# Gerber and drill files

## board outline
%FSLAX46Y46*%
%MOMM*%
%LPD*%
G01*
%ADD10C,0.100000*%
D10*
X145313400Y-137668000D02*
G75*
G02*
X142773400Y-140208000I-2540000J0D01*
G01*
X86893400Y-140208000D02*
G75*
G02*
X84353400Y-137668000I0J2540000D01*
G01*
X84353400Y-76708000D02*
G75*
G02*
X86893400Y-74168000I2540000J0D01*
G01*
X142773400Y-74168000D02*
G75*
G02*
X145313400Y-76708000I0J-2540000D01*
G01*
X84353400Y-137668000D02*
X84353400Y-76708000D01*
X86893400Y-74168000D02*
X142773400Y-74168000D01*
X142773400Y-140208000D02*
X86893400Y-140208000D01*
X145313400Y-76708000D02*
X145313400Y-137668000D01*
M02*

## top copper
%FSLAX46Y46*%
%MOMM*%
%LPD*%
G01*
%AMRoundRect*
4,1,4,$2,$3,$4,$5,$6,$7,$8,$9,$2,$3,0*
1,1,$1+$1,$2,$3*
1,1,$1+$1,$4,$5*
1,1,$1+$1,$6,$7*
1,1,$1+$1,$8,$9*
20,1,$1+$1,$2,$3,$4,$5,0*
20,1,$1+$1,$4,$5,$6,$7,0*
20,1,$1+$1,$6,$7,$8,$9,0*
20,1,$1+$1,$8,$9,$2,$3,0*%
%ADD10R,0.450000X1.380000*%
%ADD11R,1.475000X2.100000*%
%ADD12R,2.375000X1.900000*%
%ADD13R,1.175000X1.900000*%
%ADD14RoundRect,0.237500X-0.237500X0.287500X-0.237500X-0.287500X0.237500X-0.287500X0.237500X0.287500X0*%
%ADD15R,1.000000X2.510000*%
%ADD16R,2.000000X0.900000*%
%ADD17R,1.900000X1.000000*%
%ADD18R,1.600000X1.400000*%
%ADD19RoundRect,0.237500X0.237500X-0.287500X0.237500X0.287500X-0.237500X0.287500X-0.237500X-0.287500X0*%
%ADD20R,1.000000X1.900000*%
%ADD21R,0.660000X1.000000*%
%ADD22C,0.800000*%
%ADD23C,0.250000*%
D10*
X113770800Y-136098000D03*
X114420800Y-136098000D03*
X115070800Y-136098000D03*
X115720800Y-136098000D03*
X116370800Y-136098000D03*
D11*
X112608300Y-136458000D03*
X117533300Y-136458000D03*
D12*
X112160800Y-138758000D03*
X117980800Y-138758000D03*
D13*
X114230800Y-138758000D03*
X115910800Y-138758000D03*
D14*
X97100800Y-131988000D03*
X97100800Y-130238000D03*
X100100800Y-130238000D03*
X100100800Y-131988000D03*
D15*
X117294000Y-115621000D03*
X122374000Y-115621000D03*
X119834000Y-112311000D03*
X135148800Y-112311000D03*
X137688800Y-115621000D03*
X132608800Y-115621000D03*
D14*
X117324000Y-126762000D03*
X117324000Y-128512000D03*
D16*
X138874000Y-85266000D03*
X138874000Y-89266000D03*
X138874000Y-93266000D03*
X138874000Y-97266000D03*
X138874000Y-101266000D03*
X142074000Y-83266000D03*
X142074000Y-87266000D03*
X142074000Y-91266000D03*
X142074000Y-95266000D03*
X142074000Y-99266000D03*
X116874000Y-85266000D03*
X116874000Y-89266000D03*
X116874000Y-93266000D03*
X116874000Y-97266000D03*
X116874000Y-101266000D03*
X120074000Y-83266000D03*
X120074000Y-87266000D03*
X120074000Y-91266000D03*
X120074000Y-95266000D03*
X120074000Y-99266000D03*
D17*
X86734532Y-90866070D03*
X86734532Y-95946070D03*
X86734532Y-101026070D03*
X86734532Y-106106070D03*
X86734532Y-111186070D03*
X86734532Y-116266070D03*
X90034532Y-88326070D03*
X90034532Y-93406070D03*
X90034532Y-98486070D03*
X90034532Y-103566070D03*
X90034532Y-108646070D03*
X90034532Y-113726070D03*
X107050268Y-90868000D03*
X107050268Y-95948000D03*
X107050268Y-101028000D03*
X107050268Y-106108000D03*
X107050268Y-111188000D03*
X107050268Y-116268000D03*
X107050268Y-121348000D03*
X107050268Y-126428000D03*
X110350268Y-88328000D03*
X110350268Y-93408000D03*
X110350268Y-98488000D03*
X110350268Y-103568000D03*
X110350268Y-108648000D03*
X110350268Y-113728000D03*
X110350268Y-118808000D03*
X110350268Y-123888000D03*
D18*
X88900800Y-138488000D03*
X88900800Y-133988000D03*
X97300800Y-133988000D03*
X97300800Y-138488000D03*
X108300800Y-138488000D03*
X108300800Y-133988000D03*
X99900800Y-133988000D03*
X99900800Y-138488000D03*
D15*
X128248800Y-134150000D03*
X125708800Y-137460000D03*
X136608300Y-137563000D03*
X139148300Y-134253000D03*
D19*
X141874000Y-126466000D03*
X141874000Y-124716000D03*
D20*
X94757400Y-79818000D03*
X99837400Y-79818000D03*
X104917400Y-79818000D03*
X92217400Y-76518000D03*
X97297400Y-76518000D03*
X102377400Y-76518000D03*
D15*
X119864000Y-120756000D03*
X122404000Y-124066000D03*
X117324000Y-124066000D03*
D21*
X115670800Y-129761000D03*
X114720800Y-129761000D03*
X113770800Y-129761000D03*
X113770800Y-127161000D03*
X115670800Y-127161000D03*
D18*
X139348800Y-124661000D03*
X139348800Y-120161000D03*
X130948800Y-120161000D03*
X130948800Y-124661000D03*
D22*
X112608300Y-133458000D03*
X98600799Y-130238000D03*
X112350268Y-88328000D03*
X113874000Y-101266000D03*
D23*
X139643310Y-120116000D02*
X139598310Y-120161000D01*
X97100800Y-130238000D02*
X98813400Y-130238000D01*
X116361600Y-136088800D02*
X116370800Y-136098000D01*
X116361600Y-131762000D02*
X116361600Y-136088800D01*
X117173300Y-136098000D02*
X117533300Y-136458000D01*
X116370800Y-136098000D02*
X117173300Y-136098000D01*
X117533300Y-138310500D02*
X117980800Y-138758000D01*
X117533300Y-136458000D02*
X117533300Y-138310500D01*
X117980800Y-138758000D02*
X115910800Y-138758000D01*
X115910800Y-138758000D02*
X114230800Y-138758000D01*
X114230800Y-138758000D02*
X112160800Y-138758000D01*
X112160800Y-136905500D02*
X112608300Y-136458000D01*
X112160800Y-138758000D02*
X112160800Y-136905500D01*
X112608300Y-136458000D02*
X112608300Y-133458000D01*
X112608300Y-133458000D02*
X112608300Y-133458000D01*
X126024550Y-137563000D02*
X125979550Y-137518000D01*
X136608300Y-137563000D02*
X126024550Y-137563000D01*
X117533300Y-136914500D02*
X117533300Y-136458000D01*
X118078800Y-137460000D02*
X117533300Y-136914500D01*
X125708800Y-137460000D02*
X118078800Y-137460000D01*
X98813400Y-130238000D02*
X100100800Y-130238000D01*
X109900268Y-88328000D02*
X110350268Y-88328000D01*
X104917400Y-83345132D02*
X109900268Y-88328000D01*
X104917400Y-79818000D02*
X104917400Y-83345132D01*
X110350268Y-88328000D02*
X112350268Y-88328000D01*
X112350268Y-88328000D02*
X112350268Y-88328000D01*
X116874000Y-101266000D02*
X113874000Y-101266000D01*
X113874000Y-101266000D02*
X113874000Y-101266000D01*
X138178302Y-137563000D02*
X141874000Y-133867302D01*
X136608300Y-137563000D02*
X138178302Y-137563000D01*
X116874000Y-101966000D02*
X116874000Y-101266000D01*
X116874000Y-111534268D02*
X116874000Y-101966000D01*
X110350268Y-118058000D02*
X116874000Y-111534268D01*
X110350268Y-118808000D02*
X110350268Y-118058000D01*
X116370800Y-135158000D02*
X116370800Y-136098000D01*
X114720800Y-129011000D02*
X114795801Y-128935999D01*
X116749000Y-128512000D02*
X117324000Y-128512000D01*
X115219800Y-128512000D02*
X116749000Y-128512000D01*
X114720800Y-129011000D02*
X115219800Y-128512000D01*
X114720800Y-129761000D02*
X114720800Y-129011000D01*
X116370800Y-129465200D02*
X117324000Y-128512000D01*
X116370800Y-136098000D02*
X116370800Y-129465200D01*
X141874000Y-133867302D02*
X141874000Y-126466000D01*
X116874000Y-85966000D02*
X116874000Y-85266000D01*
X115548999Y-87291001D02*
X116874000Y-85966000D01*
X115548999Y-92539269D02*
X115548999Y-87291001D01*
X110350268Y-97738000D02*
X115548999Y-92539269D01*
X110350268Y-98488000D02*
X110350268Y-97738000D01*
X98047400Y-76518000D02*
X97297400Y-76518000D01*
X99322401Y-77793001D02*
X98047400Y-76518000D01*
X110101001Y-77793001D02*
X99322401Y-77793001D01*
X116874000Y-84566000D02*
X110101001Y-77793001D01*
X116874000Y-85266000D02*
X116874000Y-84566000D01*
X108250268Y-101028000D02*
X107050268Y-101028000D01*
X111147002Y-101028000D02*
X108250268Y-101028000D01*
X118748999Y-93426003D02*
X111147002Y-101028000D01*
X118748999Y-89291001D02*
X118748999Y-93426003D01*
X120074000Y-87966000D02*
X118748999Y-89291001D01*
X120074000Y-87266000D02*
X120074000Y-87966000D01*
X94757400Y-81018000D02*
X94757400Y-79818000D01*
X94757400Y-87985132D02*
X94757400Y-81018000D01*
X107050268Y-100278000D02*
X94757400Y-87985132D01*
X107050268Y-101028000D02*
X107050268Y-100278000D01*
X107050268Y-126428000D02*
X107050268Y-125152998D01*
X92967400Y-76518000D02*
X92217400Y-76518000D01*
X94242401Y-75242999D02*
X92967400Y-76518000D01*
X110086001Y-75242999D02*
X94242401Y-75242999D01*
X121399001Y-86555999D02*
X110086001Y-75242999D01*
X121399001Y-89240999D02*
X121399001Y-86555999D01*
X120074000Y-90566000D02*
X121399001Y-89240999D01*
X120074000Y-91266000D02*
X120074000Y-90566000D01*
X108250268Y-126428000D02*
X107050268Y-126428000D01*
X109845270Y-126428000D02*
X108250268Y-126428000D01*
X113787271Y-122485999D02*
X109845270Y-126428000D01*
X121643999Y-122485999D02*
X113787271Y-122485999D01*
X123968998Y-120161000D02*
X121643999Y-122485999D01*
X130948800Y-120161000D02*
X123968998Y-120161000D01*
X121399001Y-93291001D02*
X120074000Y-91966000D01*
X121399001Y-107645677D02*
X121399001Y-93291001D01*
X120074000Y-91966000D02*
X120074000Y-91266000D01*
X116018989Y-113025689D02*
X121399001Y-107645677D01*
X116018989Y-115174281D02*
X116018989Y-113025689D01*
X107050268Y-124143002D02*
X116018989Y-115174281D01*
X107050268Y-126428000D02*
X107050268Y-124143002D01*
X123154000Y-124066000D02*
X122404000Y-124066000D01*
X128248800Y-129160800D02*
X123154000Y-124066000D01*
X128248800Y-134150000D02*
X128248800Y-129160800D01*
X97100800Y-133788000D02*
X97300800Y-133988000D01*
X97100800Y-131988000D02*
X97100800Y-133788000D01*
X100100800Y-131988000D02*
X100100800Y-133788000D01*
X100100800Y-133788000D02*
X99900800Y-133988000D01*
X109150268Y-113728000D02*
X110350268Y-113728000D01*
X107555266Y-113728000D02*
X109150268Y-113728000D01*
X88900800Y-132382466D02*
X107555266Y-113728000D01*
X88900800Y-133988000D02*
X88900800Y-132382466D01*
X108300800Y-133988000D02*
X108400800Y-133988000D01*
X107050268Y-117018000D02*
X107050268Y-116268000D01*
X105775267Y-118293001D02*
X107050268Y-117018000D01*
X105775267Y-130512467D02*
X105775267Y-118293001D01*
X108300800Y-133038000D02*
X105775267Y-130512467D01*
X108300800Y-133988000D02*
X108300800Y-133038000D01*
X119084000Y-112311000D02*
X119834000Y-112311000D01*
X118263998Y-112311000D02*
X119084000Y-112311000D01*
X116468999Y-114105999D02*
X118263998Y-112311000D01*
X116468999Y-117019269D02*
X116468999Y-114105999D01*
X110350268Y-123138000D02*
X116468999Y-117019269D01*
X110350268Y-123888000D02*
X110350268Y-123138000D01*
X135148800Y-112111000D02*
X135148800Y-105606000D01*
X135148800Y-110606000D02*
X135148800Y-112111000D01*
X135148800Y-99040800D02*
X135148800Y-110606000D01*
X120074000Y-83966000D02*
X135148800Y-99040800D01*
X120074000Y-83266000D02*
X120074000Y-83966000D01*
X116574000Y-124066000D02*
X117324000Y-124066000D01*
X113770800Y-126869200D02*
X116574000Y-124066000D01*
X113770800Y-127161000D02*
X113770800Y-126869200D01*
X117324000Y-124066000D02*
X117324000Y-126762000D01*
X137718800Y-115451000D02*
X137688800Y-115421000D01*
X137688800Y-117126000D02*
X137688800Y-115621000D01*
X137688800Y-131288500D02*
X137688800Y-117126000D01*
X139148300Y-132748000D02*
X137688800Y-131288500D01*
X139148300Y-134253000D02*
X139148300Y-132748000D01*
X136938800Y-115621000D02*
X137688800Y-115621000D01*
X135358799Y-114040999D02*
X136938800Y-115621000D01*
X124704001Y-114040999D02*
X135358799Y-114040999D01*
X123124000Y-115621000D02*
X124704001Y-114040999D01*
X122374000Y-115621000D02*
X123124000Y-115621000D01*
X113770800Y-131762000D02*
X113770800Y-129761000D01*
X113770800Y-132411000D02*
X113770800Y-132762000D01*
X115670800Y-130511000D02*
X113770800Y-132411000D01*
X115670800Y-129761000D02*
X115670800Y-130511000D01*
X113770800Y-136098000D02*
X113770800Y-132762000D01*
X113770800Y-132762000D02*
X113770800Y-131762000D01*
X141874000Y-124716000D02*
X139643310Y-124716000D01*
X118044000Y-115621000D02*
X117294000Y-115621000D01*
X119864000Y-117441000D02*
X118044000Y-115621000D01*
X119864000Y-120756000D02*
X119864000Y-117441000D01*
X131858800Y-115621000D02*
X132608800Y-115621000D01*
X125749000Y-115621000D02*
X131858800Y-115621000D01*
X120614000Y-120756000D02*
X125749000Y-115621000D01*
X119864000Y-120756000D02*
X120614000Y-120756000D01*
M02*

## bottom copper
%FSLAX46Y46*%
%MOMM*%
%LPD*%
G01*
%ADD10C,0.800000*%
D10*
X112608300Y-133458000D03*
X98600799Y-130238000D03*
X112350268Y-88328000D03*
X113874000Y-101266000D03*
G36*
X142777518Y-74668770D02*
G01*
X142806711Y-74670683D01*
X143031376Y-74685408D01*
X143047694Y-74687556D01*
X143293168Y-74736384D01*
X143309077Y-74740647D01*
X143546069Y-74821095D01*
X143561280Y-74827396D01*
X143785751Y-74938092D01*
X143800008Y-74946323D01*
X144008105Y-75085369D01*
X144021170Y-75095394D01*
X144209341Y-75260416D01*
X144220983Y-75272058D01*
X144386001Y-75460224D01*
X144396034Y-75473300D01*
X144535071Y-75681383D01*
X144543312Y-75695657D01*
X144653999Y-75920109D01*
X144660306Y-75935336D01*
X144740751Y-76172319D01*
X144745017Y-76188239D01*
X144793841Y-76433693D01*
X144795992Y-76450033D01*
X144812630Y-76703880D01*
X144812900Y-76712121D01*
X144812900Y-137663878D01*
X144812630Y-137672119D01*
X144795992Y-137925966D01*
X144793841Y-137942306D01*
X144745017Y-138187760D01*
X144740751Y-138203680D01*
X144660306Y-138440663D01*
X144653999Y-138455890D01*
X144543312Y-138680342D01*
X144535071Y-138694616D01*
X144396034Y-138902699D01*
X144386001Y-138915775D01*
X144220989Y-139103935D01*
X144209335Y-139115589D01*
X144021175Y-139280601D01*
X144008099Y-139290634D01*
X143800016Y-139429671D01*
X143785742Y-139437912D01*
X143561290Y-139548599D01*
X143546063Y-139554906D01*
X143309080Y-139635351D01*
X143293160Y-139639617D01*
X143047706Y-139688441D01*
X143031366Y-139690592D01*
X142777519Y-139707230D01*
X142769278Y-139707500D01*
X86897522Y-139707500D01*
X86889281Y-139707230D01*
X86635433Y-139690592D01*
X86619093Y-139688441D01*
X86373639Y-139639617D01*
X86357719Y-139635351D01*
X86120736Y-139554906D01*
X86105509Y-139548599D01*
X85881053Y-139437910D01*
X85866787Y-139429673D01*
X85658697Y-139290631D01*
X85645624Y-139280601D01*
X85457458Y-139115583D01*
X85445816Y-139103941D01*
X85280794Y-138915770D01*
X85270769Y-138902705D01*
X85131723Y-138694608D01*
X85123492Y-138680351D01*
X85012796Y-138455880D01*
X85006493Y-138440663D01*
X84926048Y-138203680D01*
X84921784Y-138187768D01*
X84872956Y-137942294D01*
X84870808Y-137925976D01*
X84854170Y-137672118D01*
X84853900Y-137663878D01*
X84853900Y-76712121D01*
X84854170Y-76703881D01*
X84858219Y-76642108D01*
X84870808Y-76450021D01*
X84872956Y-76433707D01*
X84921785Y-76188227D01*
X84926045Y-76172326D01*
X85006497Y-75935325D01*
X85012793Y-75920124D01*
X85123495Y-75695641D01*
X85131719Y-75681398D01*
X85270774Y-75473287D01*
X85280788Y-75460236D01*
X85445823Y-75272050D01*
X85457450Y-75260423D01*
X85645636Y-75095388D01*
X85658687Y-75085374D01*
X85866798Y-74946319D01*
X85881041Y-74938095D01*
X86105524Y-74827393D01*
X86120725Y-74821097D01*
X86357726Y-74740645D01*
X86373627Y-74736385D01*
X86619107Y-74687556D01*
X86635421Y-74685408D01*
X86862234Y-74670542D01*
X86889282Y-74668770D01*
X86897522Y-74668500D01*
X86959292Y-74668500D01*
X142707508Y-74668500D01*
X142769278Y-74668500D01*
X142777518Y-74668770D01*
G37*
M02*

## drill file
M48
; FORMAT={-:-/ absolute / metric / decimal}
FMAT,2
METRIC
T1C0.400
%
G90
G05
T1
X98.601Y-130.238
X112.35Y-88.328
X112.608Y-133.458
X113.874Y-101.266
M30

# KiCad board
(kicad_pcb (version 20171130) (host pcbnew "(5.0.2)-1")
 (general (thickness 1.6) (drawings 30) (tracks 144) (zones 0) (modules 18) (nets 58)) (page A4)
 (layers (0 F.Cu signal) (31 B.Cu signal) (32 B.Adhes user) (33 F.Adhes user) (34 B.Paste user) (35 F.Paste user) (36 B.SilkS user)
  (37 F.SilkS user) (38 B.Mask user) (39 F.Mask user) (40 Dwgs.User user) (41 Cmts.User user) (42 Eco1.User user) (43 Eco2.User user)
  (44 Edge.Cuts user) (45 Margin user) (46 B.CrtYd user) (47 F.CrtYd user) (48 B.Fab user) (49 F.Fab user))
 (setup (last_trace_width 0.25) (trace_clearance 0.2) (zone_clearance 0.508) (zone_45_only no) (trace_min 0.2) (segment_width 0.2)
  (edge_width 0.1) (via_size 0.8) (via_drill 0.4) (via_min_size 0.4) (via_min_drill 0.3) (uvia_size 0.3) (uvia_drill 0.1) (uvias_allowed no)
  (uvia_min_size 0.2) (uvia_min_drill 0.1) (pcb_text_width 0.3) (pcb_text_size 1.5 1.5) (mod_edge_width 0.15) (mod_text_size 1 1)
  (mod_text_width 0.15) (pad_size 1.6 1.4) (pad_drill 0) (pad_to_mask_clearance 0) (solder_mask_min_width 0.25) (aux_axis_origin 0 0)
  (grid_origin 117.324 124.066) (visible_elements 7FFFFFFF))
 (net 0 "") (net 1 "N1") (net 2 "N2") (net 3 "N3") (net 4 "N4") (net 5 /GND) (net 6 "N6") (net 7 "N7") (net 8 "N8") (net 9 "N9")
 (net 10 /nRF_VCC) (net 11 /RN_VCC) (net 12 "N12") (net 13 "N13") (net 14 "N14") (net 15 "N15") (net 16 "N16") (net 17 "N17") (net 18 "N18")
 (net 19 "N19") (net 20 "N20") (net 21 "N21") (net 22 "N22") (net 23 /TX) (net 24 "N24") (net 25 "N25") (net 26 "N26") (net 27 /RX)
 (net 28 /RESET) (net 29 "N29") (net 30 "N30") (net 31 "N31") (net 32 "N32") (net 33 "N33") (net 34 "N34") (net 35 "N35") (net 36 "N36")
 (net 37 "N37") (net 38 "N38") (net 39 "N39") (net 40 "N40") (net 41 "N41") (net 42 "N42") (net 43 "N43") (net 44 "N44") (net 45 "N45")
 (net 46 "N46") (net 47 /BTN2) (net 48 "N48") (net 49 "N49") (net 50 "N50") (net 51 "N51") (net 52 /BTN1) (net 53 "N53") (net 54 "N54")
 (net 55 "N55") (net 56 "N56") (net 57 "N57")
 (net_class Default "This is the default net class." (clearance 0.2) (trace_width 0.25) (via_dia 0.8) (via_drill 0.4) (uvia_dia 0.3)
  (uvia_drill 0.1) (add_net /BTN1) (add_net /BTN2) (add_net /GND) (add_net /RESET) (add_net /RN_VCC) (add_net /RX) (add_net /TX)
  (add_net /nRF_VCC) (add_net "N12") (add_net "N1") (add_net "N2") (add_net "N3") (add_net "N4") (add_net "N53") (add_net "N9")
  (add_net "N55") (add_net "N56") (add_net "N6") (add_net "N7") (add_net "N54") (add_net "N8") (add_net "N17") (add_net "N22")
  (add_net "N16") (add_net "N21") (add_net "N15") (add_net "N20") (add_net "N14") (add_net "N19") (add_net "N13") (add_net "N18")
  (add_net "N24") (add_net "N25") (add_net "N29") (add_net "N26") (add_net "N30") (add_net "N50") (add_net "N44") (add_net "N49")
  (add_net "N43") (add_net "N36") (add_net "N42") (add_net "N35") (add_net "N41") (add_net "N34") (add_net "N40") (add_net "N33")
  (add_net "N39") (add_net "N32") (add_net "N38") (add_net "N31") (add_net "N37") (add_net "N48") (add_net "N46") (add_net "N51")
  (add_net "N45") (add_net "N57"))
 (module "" (layer F.Cu) (at 106.3244 75.50912)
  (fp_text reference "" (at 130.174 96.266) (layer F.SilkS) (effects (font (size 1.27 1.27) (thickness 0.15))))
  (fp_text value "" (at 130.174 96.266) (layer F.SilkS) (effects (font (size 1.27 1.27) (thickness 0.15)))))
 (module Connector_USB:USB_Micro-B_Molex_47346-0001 (layer F.Cu) (at 115.0708 137.558)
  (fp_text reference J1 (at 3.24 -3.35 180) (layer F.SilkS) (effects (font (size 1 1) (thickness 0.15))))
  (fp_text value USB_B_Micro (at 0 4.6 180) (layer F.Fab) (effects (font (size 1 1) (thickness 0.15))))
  (pad 1 smd rect (at -1.3 -1.46) (size 0.45 1.38) (layers F.Cu F.Paste F.Mask) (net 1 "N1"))
  (pad 2 smd rect (at -0.65 -1.46) (size 0.45 1.38) (layers F.Cu F.Paste F.Mask) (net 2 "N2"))
  (pad 3 smd rect (at 0 -1.46) (size 0.45 1.38) (layers F.Cu F.Paste F.Mask) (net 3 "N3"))
  (pad 4 smd rect (at 0.65 -1.46) (size 0.45 1.38) (layers F.Cu F.Paste F.Mask) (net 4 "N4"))
  (pad 5 smd rect (at 1.3 -1.46) (size 0.45 1.38) (layers F.Cu F.Paste F.Mask) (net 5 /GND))
  (pad 6 smd rect (at -2.4625 -1.1) (size 1.475 2.1) (layers F.Cu F.Paste F.Mask) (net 5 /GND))
  (pad 6 smd rect (at 2.4625 -1.1) (size 1.475 2.1) (layers F.Cu F.Paste F.Mask) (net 5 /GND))
  (pad 6 smd rect (at -2.91 1.2) (size 2.375 1.9) (layers F.Cu F.Paste F.Mask) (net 5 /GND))
  (pad 6 smd rect (at 2.91 1.2) (size 2.375 1.9) (layers F.Cu F.Paste F.Mask) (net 5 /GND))
  (pad 6 smd rect (at -0.84 1.2) (size 1.175 1.9) (layers F.Cu F.Paste F.Mask) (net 5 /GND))
  (pad 6 smd rect (at 0.84 1.2) (size 1.175 1.9) (layers F.Cu F.Paste F.Mask) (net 5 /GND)))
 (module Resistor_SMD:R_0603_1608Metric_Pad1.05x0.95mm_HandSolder (layer F.Cu) (at 97.1008 131.113 270)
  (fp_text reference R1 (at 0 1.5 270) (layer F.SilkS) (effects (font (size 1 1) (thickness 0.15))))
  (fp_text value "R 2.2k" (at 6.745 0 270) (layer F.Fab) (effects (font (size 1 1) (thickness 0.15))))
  (pad 2 smd roundrect (at 0.875 0 270) (size 1.05 0.95) (layers F.Cu F.Paste F.Mask) (roundrect_rratio 0.25) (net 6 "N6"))
  (pad 1 smd roundrect (at -0.875 0 270) (size 1.05 0.95) (layers F.Cu F.Paste F.Mask) (roundrect_rratio 0.25) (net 5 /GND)))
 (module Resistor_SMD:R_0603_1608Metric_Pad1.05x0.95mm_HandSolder (layer F.Cu) (at 100.1008 131.113 270)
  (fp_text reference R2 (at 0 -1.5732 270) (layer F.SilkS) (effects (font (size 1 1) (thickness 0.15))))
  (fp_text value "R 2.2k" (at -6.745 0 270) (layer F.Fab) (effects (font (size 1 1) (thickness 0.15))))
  (pad 1 smd roundrect (at -0.875 0 270) (size 1.05 0.95) (layers F.Cu F.Paste F.Mask) (roundrect_rratio 0.25) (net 5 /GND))
  (pad 2 smd roundrect (at 0.875 0 270) (size 1.05 0.95) (layers F.Cu F.Paste F.Mask) (roundrect_rratio 0.25) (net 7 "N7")))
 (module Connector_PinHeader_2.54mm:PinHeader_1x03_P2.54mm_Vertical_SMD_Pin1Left (layer F.Cu) (at 119.834 113.966 90)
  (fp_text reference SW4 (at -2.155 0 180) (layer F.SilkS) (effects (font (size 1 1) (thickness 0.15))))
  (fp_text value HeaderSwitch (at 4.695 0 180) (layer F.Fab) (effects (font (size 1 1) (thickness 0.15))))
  (pad 1 smd rect (at -1.655 -2.54 90) (size 2.51 1) (layers F.Cu F.Paste F.Mask) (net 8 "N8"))
  (pad 3 smd rect (at -1.655 2.54 90) (size 2.51 1) (layers F.Cu F.Paste F.Mask) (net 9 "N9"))
  (pad 2 smd rect (at 1.655 0 90) (size 2.51 1) (layers F.Cu F.Paste F.Mask) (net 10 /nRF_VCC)))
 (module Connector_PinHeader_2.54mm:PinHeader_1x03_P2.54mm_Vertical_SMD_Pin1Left (layer F.Cu) (at 135.1488 113.966 90)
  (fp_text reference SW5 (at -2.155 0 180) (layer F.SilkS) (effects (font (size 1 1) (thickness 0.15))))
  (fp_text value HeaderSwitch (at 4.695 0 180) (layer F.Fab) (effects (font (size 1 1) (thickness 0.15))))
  (pad 2 smd rect (at 1.655 0 90) (size 2.51 1) (layers F.Cu F.Paste F.Mask) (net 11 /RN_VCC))
  (pad 3 smd rect (at -1.655 2.54 90) (size 2.51 1) (layers F.Cu F.Paste F.Mask) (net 9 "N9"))
  (pad 1 smd rect (at -1.655 -2.54 90) (size 2.51 1) (layers F.Cu F.Paste F.Mask) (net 8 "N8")))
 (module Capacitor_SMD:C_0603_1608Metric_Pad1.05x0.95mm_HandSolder (layer F.Cu) (at 117.324 127.637 270)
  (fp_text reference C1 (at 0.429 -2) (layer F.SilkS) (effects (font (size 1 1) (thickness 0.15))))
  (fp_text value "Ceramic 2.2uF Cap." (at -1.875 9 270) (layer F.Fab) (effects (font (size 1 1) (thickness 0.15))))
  (pad 1 smd roundrect (at -0.875 0 270) (size 1.05 0.95) (layers F.Cu F.Paste F.Mask) (roundrect_rratio 0.25) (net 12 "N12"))
  (pad 2 smd roundrect (at 0.875 0 270) (size 1.05 0.95) (layers F.Cu F.Paste F.Mask) (roundrect_rratio 0.25) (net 5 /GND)))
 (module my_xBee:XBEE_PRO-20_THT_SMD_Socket (layer F.Cu) (at 129.474 95.266)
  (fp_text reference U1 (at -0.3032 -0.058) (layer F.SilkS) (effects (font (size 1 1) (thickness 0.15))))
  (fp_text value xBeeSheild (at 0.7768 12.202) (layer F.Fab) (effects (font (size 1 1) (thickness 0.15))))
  (pad 19 smd rect (at 9.4 -10) (size 2 0.9) (layers F.Cu F.Paste F.Mask) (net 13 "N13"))
  (pad 17 smd rect (at 9.4 -6) (size 2 0.9) (layers F.Cu F.Paste F.Mask) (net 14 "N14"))
  (pad 15 smd rect (at 9.4 -2) (size 2 0.9) (layers F.Cu F.Paste F.Mask) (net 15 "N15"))
  (pad 13 smd rect (at 9.4 2) (size 2 0.9) (layers F.Cu F.Paste F.Mask) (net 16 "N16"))
  (pad 11 smd rect (at 9.4 6) (size 2 0.9) (layers F.Cu F.Paste F.Mask) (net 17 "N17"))
  (pad 20 smd rect (at 12.6 -12) (size 2 0.9) (layers F.Cu F.Paste F.Mask) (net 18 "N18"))
  (pad 18 smd rect (at 12.6 -8) (size 2 0.9) (layers F.Cu F.Paste F.Mask) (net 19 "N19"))
  (pad 16 smd rect (at 12.6 -4) (size 2 0.9) (layers F.Cu F.Paste F.Mask) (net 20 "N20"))
  (pad 14 smd rect (at 12.6 0) (size 2 0.9) (layers F.Cu F.Paste F.Mask) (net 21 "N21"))
  (pad 12 smd rect (at 12.6 4) (size 2 0.9) (layers F.Cu F.Paste F.Mask) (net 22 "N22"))
  (pad 2 smd rect (at -12.6 -10) (size 2 0.9) (layers F.Cu F.Paste F.Mask) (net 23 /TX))
  (pad 4 smd rect (at -12.6 -6) (size 2 0.9) (layers F.Cu F.Paste F.Mask) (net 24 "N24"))
  (pad 6 smd rect (at -12.6 -2) (size 2 0.9) (layers F.Cu F.Paste F.Mask) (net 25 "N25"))
  (pad 8 smd rect (at -12.6 2) (size 2 0.9) (layers F.Cu F.Paste F.Mask) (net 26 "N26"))
  (pad 10 smd rect (at -12.6 6) (size 2 0.9) (layers F.Cu F.Paste F.Mask) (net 5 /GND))
  (pad 1 smd rect (at -9.4 -12) (size 2 0.9) (layers F.Cu F.Paste F.Mask) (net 11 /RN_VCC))
  (pad 3 smd rect (at -9.4 -8) (size 2 0.9) (layers F.Cu F.Paste F.Mask) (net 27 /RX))
  (pad 5 smd rect (at -9.4 -4) (size 2 0.9) (layers F.Cu F.Paste F.Mask) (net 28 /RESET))
  (pad 7 smd rect (at -9.4 0) (size 2 0.9) (layers F.Cu F.Paste F.Mask) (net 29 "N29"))
  (pad 9 smd rect (at -9.4 4) (size 2 0.9) (layers F.Cu F.Paste F.Mask) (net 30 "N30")))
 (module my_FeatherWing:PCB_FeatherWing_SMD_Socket (layer F.Cu) (at 99.022868 107.378 90)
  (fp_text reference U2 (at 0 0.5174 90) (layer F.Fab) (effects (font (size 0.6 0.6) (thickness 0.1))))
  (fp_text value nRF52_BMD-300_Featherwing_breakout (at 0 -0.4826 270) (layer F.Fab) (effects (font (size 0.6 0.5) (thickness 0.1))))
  (pad 27 smd rect (at 16.51193 -12.288336 180) (size 1.9 1) (layers F.Cu F.Paste F.Mask) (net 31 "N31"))
  (pad 25 smd rect (at 11.43193 -12.288336 180) (size 1.9 1) (layers F.Cu F.Paste F.Mask) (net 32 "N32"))
  (pad 23 smd rect (at 6.35193 -12.288336 180) (size 1.9 1) (layers F.Cu F.Paste F.Mask) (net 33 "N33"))
  (pad 21 smd rect (at 1.27193 -12.288336 180) (size 1.9 1) (layers F.Cu F.Paste F.Mask) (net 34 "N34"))
  (pad 19 smd rect (at -3.80807 -12.288336 180) (size 1.9 1) (layers F.Cu F.Paste F.Mask) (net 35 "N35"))
  (pad 17 smd rect (at -8.88807 -12.288336 180) (size 1.9 1) (layers F.Cu F.Paste F.Mask) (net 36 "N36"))
  (pad 28 smd rect (at 19.05193 -8.988336 180) (size 1.9 1) (layers F.Cu F.Paste F.Mask) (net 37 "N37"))
  (pad 26 smd rect (at 13.97193 -8.988336 180) (size 1.9 1) (layers F.Cu F.Paste F.Mask) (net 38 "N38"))
  (pad 24 smd rect (at 8.89193 -8.988336 180) (size 1.9 1) (layers F.Cu F.Paste F.Mask) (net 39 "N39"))
  (pad 22 smd rect (at 3.81193 -8.988336 180) (size 1.9 1) (layers F.Cu F.Paste F.Mask) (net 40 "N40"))
  (pad 20 smd rect (at -1.26807 -8.988336 180) (size 1.9 1) (layers F.Cu F.Paste F.Mask) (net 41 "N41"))
  (pad 18 smd rect (at -6.34807 -8.988336 180) (size 1.9 1) (layers F.Cu F.Paste F.Mask) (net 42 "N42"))
  (pad 15 smd rect (at 16.51 8.0274 180) (size 1.9 1) (layers F.Cu F.Paste F.Mask) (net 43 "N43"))
  (pad 13 smd rect (at 11.43 8.0274 180) (size 1.9 1) (layers F.Cu F.Paste F.Mask) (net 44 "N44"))
  (pad 11 smd rect (at 6.35 8.0274 180) (size 1.9 1) (layers F.Cu F.Paste F.Mask) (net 27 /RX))
  (pad 9 smd rect (at 1.27 8.0274 180) (size 1.9 1) (layers F.Cu F.Paste F.Mask) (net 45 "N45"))
  (pad 7 smd rect (at -3.81 8.0274 180) (size 1.9 1) (layers F.Cu F.Paste F.Mask) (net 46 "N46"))
  (pad 5 smd rect (at -8.89 8.0274 180) (size 1.9 1) (layers F.Cu F.Paste F.Mask) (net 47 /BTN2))
  (pad 3 smd rect (at -13.97 8.0274 180) (size 1.9 1) (layers F.Cu F.Paste F.Mask) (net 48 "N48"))
  (pad 1 smd rect (at -19.05 8.0274 180) (size 1.9 1) (layers F.Cu F.Paste F.Mask) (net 28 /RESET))
  (pad 16 smd rect (at 19.05 11.3274 180) (size 1.9 1) (layers F.Cu F.Paste F.Mask) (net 5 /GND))
  (pad 14 smd rect (at 13.97 11.3274 180) (size 1.9 1) (layers F.Cu F.Paste F.Mask) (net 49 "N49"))
  (pad 12 smd rect (at 8.89 11.3274 180) (size 1.9 1) (layers F.Cu F.Paste F.Mask) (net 23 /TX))
  (pad 10 smd rect (at 3.81 11.3274 180) (size 1.9 1) (layers F.Cu F.Paste F.Mask) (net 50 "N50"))
  (pad 8 smd rect (at -1.27 11.3274 180) (size 1.9 1) (layers F.Cu F.Paste F.Mask) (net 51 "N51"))
  (pad 6 smd rect (at -6.35 11.3274 180) (size 1.9 1) (layers F.Cu F.Paste F.Mask) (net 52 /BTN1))
  (pad 4 smd rect (at -11.43 11.3274 180) (size 1.9 1) (layers F.Cu F.Paste F.Mask) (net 5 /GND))
  (pad 2 smd rect (at -16.51 11.3274 180) (size 1.9 1) (layers F.Cu F.Paste F.Mask) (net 10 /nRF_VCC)))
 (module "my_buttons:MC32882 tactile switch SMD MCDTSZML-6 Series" (layer F.Cu) (at 93.1008 136.238)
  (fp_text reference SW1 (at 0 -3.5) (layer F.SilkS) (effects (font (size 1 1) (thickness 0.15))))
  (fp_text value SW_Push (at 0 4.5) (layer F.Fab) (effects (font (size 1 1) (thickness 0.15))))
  (pad 3 smd rect (at -4.2 2.25) (size 1.6 1.4) (layers F.Cu F.Paste F.Mask))
  (pad 1 smd rect (at -4.2 -2.25) (size 1.6 1.4) (layers F.Cu F.Paste F.Mask) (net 52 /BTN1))
  (pad 2 smd rect (at 4.2 -2.25) (size 1.6 1.4) (layers F.Cu F.Paste F.Mask) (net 6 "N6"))
  (pad 4 smd rect (at 4.2 2.25) (size 1.6 1.4) (layers F.Cu F.Paste F.Mask)))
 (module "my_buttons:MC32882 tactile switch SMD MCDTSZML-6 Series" (layer F.Cu) (at 104.1008 136.238)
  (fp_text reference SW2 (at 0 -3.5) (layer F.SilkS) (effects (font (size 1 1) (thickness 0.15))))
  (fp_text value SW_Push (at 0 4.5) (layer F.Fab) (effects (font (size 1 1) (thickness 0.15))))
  (pad 4 smd rect (at 4.2 2.25) (size 1.6 1.4) (layers F.Cu F.Paste F.Mask))
  (pad 2 smd rect (at 4.2 -2.25) (size 1.6 1.4) (layers F.Cu F.Paste F.Mask) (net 47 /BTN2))
  (pad 1 smd rect (at -4.2 -2.25) (size 1.6 1.4) (layers F.Cu F.Paste F.Mask) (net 7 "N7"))
  (pad 3 smd rect (at -4.2 2.25) (size 1.6 1.4) (layers F.Cu F.Paste F.Mask)))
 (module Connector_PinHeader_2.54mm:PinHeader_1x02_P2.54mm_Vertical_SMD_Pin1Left (layer F.Cu) (at 126.9788 135.805 270)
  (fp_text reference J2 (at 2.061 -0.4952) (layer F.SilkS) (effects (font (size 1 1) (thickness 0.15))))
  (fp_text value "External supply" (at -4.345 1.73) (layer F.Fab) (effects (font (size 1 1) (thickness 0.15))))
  (pad 1 smd rect (at -1.655 -1.27 270) (size 2.51 1) (layers F.Cu F.Paste F.Mask) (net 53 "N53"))
  (pad 2 smd rect (at 1.655 1.27 270) (size 2.51 1) (layers F.Cu F.Paste F.Mask) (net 5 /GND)))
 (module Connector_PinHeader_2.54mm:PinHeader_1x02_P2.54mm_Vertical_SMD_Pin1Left (layer F.Cu) (at 137.8783 135.908 270)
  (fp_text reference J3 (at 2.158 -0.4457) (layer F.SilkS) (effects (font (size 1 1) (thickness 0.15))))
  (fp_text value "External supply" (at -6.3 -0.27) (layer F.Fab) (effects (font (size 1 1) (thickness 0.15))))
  (pad 2 smd rect (at 1.655 1.27 270) (size 2.51 1) (layers F.Cu F.Paste F.Mask) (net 5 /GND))
  (pad 1 smd rect (at -1.655 -1.27 270) (size 2.51 1) (layers F.Cu F.Paste F.Mask) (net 9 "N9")))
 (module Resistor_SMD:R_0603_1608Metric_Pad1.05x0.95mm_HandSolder (layer F.Cu) (at 141.874 125.591 90)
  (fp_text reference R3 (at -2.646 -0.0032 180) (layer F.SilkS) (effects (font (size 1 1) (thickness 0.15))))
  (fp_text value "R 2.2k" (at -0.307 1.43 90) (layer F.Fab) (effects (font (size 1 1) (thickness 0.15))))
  (pad 1 smd roundrect (at -0.875 0 90) (size 1.05 0.95) (layers F.Cu F.Paste F.Mask) (roundrect_rratio 0.25) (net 5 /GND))
  (pad 2 smd roundrect (at 0.875 0 90) (size 1.05 0.95) (layers F.Cu F.Paste F.Mask) (roundrect_rratio 0.25) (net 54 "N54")))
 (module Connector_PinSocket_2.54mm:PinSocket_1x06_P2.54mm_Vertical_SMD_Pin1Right (layer F.Cu) (at 98.5674 78.168 90)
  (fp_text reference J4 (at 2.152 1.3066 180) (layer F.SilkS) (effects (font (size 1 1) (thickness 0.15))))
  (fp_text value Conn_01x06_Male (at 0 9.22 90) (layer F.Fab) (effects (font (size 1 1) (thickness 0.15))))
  (pad 2 smd rect (at -1.65 -3.81 90) (size 1.9 1) (layers F.Cu F.Paste F.Mask) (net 27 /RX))
  (pad 4 smd rect (at -1.65 1.27 90) (size 1.9 1) (layers F.Cu F.Paste F.Mask) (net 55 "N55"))
  (pad 6 smd rect (at -1.65 6.35 90) (size 1.9 1) (layers F.Cu F.Paste F.Mask) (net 5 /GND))
  (pad 1 smd rect (at 1.65 -6.35 90) (size 1.9 1) (layers F.Cu F.Paste F.Mask) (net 28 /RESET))
  (pad 3 smd rect (at 1.65 -1.27 90) (size 1.9 1) (layers F.Cu F.Paste F.Mask) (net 23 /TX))
  (pad 5 smd rect (at 1.65 3.81 90) (size 1.9 1) (layers F.Cu F.Paste F.Mask) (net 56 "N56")))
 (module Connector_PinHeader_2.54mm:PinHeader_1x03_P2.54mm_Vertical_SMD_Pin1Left (layer F.Cu) (at 119.864 122.411 90)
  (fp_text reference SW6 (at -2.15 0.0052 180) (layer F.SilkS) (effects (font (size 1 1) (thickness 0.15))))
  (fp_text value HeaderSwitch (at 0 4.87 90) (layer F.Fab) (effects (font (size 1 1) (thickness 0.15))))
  (pad 2 smd rect (at 1.655 0 90) (size 2.51 1) (layers F.Cu F.Paste F.Mask) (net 8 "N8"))
  (pad 3 smd rect (at -1.655 2.54 90) (size 2.51 1) (layers F.Cu F.Paste F.Mask) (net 53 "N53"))
  (pad 1 smd rect (at -1.655 -2.54 90) (size 2.51 1) (layers F.Cu F.Paste F.Mask) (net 12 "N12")))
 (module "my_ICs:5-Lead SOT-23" (layer F.Cu) (at 114.7208 128.411 180)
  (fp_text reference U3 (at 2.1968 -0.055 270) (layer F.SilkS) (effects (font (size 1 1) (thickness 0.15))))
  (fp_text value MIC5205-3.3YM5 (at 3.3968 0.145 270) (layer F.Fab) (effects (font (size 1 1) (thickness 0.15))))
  (pad 3 smd rect (at -0.95 -1.35 180) (size 0.66 1) (layers F.Cu F.Paste F.Mask) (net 1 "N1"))
  (pad 2 smd rect (at 0 -1.35 180) (size 0.66 1) (layers F.Cu F.Paste F.Mask) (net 5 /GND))
  (pad 1 smd rect (at 0.95 -1.35 180) (size 0.66 1) (layers F.Cu F.Paste F.Mask) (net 1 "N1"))
  (pad 5 smd rect (at 0.95 1.25 180) (size 0.66 1) (layers F.Cu F.Paste F.Mask) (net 12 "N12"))
  (pad 4 smd rect (at -0.95 1.25 180) (size 0.66 1) (layers F.Cu F.Paste F.Mask) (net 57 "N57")))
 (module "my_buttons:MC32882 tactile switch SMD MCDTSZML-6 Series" (layer F.Cu) (at 135.1488 122.411)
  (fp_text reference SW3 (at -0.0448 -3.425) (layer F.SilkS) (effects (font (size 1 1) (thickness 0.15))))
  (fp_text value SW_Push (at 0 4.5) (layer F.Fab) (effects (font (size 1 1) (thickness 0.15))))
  (pad 2 smd rect (at 4.2 2.25) (size 1.6 1.4) (layers F.Cu F.Paste F.Mask) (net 54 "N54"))
  (pad "" smd rect (at 4.2 -2.25) (size 1.6 1.4) (layers F.Cu F.Paste F.Mask))
  (pad 1 smd rect (at -4.2 -2.25) (size 1.6 1.4) (layers F.Cu F.Paste F.Mask) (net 28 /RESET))
  (pad "" smd rect (at -4.2 2.25) (size 1.6 1.4) (layers F.Cu F.Paste F.Mask)))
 (gr_arc (start 142.7734 137.668) (end 142.7734 140.208) (angle -90) (layer Edge.Cuts) (width 0.1))
 (gr_arc (start 86.8934 137.668) (end 84.3534 137.668) (angle -90) (layer Edge.Cuts) (width 0.1))
 (gr_arc (start 86.8934 76.708) (end 86.8934 74.168) (angle -90) (layer Edge.Cuts) (width 0.1))
 (gr_arc (start 142.7734 76.708) (end 145.3134 76.708) (angle -90) (layer Edge.Cuts) (width 0.1))
 (gr_line (start 84.3534 137.668) (end 84.3534 76.708) (layer Edge.Cuts) (width 0.1))
 (gr_line (start 86.8934 74.168) (end 142.7734 74.168) (layer Edge.Cuts) (width 0.1))
 (gr_line (start 142.7734 140.208) (end 86.8934 140.208) (layer Edge.Cuts) (width 0.1))
 (gr_line (start 145.3134 76.708) (end 145.3134 137.668) (layer Edge.Cuts) (width 0.1))
 (segment (start 139.64331 120.116) (end 139.59831 120.161) (width 0.25) (layer F.Cu) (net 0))
 (segment (start 97.1008 130.238) (end 98.8134 130.238) (width 0.25) (layer F.Cu) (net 5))
 (segment (start 116.3616 136.0888) (end 116.3708 136.098) (width 0.25) (layer F.Cu) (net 5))
 (segment (start 116.3616 131.762) (end 116.3616 136.0888) (width 0.25) (layer F.Cu) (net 5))
 (segment (start 117.1733 136.098) (end 117.5333 136.458) (width 0.25) (layer F.Cu) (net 5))
 (segment (start 116.3708 136.098) (end 117.1733 136.098) (width 0.25) (layer F.Cu) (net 5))
 (segment (start 117.5333 138.3105) (end 117.9808 138.758) (width 0.25) (layer F.Cu) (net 5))
 (segment (start 117.5333 136.458) (end 117.5333 138.3105) (width 0.25) (layer F.Cu) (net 5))
 (segment (start 117.9808 138.758) (end 115.9108 138.758) (width 0.25) (layer F.Cu) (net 5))
 (segment (start 115.9108 138.758) (end 114.2308 138.758) (width 0.25) (layer F.Cu) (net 5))
 (segment (start 114.2308 138.758) (end 112.1608 138.758) (width 0.25) (layer F.Cu) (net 5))
 (segment (start 112.1608 136.9055) (end 112.6083 136.458) (width 0.25) (layer F.Cu) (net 5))
 (segment (start 112.1608 138.758) (end 112.1608 136.9055) (width 0.25) (layer F.Cu) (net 5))
 (segment (start 112.6083 136.458) (end 112.6083 133.458) (width 0.25) (layer F.Cu) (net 5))
 (segment (start 112.6083 133.458) (end 112.6083 133.458) (width 0.25) (layer F.Cu) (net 5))
 (via (at 112.6083 133.458) (size 0.8) (drill 0.4) (layers F.Cu B.Cu) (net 5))
 (segment (start 126.02455 137.563) (end 125.97955 137.518) (width 0.25) (layer F.Cu) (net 5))
 (segment (start 136.6083 137.563) (end 126.02455 137.563) (width 0.25) (layer F.Cu) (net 5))
 (segment (start 117.5333 136.9145) (end 117.5333 136.458) (width 0.25) (layer F.Cu) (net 5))
 (segment (start 118.0788 137.46) (end 117.5333 136.9145) (width 0.25) (layer F.Cu) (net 5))
 (segment (start 125.7088 137.46) (end 118.0788 137.46) (width 0.25) (layer F.Cu) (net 5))
 (segment (start 98.8134 130.238) (end 100.1008 130.238) (width 0.25) (layer F.Cu) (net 5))
 (via (at 98.600799 130.238) (size 0.8) (drill 0.4) (layers F.Cu B.Cu) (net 5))
 (segment (start 109.900268 88.328) (end 110.350268 88.328) (width 0.25) (layer F.Cu) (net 5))
 (segment (start 104.9174 83.345132) (end 109.900268 88.328) (width 0.25) (layer F.Cu) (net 5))
 (segment (start 104.9174 79.818) (end 104.9174 83.345132) (width 0.25) (layer F.Cu) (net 5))
 (segment (start 110.350268 88.328) (end 112.350268 88.328) (width 0.25) (layer F.Cu) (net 5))
 (segment (start 112.350268 88.328) (end 112.350268 88.328) (width 0.25) (layer F.Cu) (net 5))
 (via (at 112.350268 88.328) (size 0.8) (drill 0.4) (layers F.Cu B.Cu) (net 5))
 (segment (start 116.874 101.266) (end 113.874 101.266) (width 0.25) (layer F.Cu) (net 5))
 (segment (start 113.874 101.266) (end 113.874 101.266) (width 0.25) (layer F.Cu) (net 5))
 (via (at 113.874 101.266) (size 0.8) (drill 0.4) (layers F.Cu B.Cu) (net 5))
 (segment (start 138.178302 137.563) (end 141.874 133.867302) (width 0.25) (layer F.Cu) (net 5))
 (segment (start 136.6083 137.563) (end 138.178302 137.563) (width 0.25) (layer F.Cu) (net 5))
 (segment (start 116.874 101.966) (end 116.874 101.266) (width 0.25) (layer F.Cu) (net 5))
 (segment (start 116.874 111.534268) (end 116.874 101.966) (width 0.25) (layer F.Cu) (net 5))
 (segment (start 110.350268 118.058) (end 116.874 111.534268) (width 0.25) (layer F.Cu) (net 5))
 (segment (start 110.350268 118.808) (end 110.350268 118.058) (width 0.25) (layer F.Cu) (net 5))
 (segment (start 116.3708 135.158) (end 116.3708 136.098) (width 0.25) (layer F.Cu) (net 5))
 (segment (start 114.7208 129.011) (end 114.795801 128.935999) (width 0.25) (layer F.Cu) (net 5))
 (segment (start 116.749 128.512) (end 117.324 128.512) (width 0.25) (layer F.Cu) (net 5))
 (segment (start 115.2198 128.512) (end 116.749 128.512) (width 0.25) (layer F.Cu) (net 5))
 (segment (start 114.7208 129.011) (end 115.2198 128.512) (width 0.25) (layer F.Cu) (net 5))
 (segment (start 114.7208 129.761) (end 114.7208 129.011) (width 0.25) (layer F.Cu) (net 5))
 (segment (start 116.3708 129.4652) (end 117.324 128.512) (width 0.25) (layer F.Cu) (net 5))
 (segment (start 116.3708 136.098) (end 116.3708 129.4652) (width 0.25) (layer F.Cu) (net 5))
 (segment (start 141.874 133.867302) (end 141.874 126.466) (width 0.25) (layer F.Cu) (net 5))
 (segment (start 116.874 85.966) (end 116.874 85.266) (width 0.25) (layer F.Cu) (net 23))
 (segment (start 115.548999 87.291001) (end 116.874 85.966) (width 0.25) (layer F.Cu) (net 23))
 (segment (start 115.548999 92.539269) (end 115.548999 87.291001) (width 0.25) (layer F.Cu) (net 23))
 (segment (start 110.350268 97.738) (end 115.548999 92.539269) (width 0.25) (layer F.Cu) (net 23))
 (segment (start 110.350268 98.488) (end 110.350268 97.738) (width 0.25) (layer F.Cu) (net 23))
 (segment (start 98.0474 76.518) (end 97.2974 76.518) (width 0.25) (layer F.Cu) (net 23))
 (segment (start 99.322401 77.793001) (end 98.0474 76.518) (width 0.25) (layer F.Cu) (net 23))
 (segment (start 110.101001 77.793001) (end 99.322401 77.793001) (width 0.25) (layer F.Cu) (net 23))
 (segment (start 116.874 84.566) (end 110.101001 77.793001) (width 0.25) (layer F.Cu) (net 23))
 (segment (start 116.874 85.266) (end 116.874 84.566) (width 0.25) (layer F.Cu) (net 23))
 (segment (start 108.250268 101.028) (end 107.050268 101.028) (width 0.25) (layer F.Cu) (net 27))
 (segment (start 111.147002 101.028) (end 108.250268 101.028) (width 0.25) (layer F.Cu) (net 27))
 (segment (start 118.748999 93.426003) (end 111.147002 101.028) (width 0.25) (layer F.Cu) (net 27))
 (segment (start 118.748999 89.291001) (end 118.748999 93.426003) (width 0.25) (layer F.Cu) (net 27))
 (segment (start 120.074 87.966) (end 118.748999 89.291001) (width 0.25) (layer F.Cu) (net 27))
 (segment (start 120.074 87.266) (end 120.074 87.966) (width 0.25) (layer F.Cu) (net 27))
 (segment (start 94.7574 81.018) (end 94.7574 79.818) (width 0.25) (layer F.Cu) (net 27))
 (segment (start 94.7574 87.985132) (end 94.7574 81.018) (width 0.25) (layer F.Cu) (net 27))
 (segment (start 107.050268 100.278) (end 94.7574 87.985132) (width 0.25) (layer F.Cu) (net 27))
 (segment (start 107.050268 101.028) (end 107.050268 100.278) (width 0.25) (layer F.Cu) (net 27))
 (segment (start 107.050268 126.428) (end 107.050268 125.152998) (width 0.25) (layer F.Cu) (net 28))
 (segment (start 92.9674 76.518) (end 92.2174 76.518) (width 0.25) (layer F.Cu) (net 28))
 (segment (start 94.242401 75.242999) (end 92.9674 76.518) (width 0.25) (layer F.Cu) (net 28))
 (segment (start 110.086001 75.242999) (end 94.242401 75.242999) (width 0.25) (layer F.Cu) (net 28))
 (segment (start 121.399001 86.555999) (end 110.086001 75.242999) (width 0.25) (layer F.Cu) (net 28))
 (segment (start 121.399001 89.240999) (end 121.399001 86.555999) (width 0.25) (layer F.Cu) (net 28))
 (segment (start 120.074 90.566) (end 121.399001 89.240999) (width 0.25) (layer F.Cu) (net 28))
 (segment (start 120.074 91.266) (end 120.074 90.566) (width 0.25) (layer F.Cu) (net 28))
 (segment (start 108.250268 126.428) (end 107.050268 126.428) (width 0.25) (layer F.Cu) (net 28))
 (segment (start 109.84527 126.428) (end 108.250268 126.428) (width 0.25) (layer F.Cu) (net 28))
 (segment (start 113.787271 122.485999) (end 109.84527 126.428) (width 0.25) (layer F.Cu) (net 28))
 (segment (start 121.643999 122.485999) (end 113.787271 122.485999) (width 0.25) (layer F.Cu) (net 28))
 (segment (start 123.968998 120.161) (end 121.643999 122.485999) (width 0.25) (layer F.Cu) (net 28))
 (segment (start 130.9488 120.161) (end 123.968998 120.161) (width 0.25) (layer F.Cu) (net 28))
 (segment (start 121.399001 93.291001) (end 120.074 91.966) (width 0.25) (layer F.Cu) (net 28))
 (segment (start 121.399001 107.645677) (end 121.399001 93.291001) (width 0.25) (layer F.Cu) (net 28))
 (segment (start 120.074 91.966) (end 120.074 91.266) (width 0.25) (layer F.Cu) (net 28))
 (segment (start 116.018989 113.025689) (end 121.399001 107.645677) (width 0.25) (layer F.Cu) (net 28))
 (segment (start 116.018989 115.174281) (end 116.018989 113.025689) (width 0.25) (layer F.Cu) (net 28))
 (segment (start 107.050268 124.143002) (end 116.018989 115.174281) (width 0.25) (layer F.Cu) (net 28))
 (segment (start 107.050268 126.428) (end 107.050268 124.143002) (width 0.25) (layer F.Cu) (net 28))
 (segment (start 123.154 124.066) (end 122.404 124.066) (width 0.25) (layer F.Cu) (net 53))
 (segment (start 128.2488 129.1608) (end 123.154 124.066) (width 0.25) (layer F.Cu) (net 53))
 (segment (start 128.2488 134.15) (end 128.2488 129.1608) (width 0.25) (layer F.Cu) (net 53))
 (segment (start 97.1008 133.788) (end 97.3008 133.988) (width 0.25) (layer F.Cu) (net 6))
 (segment (start 97.1008 131.988) (end 97.1008 133.788) (width 0.25) (layer F.Cu) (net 6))
 (segment (start 100.1008 131.988) (end 100.1008 133.788) (width 0.25) (layer F.Cu) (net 7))
 (segment (start 100.1008 133.788) (end 99.9008 133.988) (width 0.25) (layer F.Cu) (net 7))
 (segment (start 109.150268 113.728) (end 110.350268 113.728) (width 0.25) (layer F.Cu) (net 52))
 (segment (start 107.555266 113.728) (end 109.150268 113.728) (width 0.25) (layer F.Cu) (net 52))
 (segment (start 88.9008 132.382466) (end 107.555266 113.728) (width 0.25) (layer F.Cu) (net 52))
 (segment (start 88.9008 133.988) (end 88.9008 132.382466) (width 0.25) (layer F.Cu) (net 52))
 (segment (start 108.3008 133.988) (end 108.4008 133.988) (width 0.25) (layer F.Cu) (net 47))
 (segment (start 107.050268 117.018) (end 107.050268 116.268) (width 0.25) (layer F.Cu) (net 47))
 (segment (start 105.775267 118.293001) (end 107.050268 117.018) (width 0.25) (layer F.Cu) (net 47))
 (segment (start 105.775267 130.512467) (end 105.775267 118.293001) (width 0.25) (layer F.Cu) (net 47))
 (segment (start 108.3008 133.038) (end 105.775267 130.512467) (width 0.25) (layer F.Cu) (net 47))
 (segment (start 108.3008 133.988) (end 108.3008 133.038) (width 0.25) (layer F.Cu) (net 47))
 (segment (start 119.084 112.311) (end 119.834 112.311) (width 0.25) (layer F.Cu) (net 10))
 (segment (start 118.263998 112.311) (end 119.084 112.311) (width 0.25) (layer F.Cu) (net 10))
 (segment (start 116.468999 114.105999) (end 118.263998 112.311) (width 0.25) (layer F.Cu) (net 10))
 (segment (start 116.468999 117.019269) (end 116.468999 114.105999) (width 0.25) (layer F.Cu) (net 10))
 (segment (start 110.350268 123.138) (end 116.468999 117.019269) (width 0.25) (layer F.Cu) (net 10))
 (segment (start 110.350268 123.888) (end 110.350268 123.138) (width 0.25) (layer F.Cu) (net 10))
 (segment (start 135.1488 112.111) (end 135.1488 105.606) (width 0.25) (layer F.Cu) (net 11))
 (segment (start 135.1488 110.606) (end 135.1488 112.111) (width 0.25) (layer F.Cu) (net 11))
 (segment (start 135.1488 99.0408) (end 135.1488 110.606) (width 0.25) (layer F.Cu) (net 11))
 (segment (start 120.074 83.966) (end 135.1488 99.0408) (width 0.25) (layer F.Cu) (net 11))
 (segment (start 120.074 83.266) (end 120.074 83.966) (width 0.25) (layer F.Cu) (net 11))
 (segment (start 116.574 124.066) (end 117.324 124.066) (width 0.25) (layer F.Cu) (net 12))
 (segment (start 113.7708 126.8692) (end 116.574 124.066) (width 0.25) (layer F.Cu) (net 12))
 (segment (start 113.7708 127.161) (end 113.7708 126.8692) (width 0.25) (layer F.Cu) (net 12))
 (segment (start 117.324 124.066) (end 117.324 126.762) (width 0.25) (layer F.Cu) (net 12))
 (segment (start 137.7188 115.451) (end 137.6888 115.421) (width 0.25) (layer F.Cu) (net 9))
 (segment (start 137.6888 117.126) (end 137.6888 115.621) (width 0.25) (layer F.Cu) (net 9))
 (segment (start 137.6888 131.2885) (end 137.6888 117.126) (width 0.25) (layer F.Cu) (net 9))
 (segment (start 139.1483 132.748) (end 137.6888 131.2885) (width 0.25) (layer F.Cu) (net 9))
 (segment (start 139.1483 134.253) (end 139.1483 132.748) (width 0.25) (layer F.Cu) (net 9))
 (segment (start 136.9388 115.621) (end 137.6888 115.621) (width 0.25) (layer F.Cu) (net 9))
 (segment (start 135.358799 114.040999) (end 136.9388 115.621) (width 0.25) (layer F.Cu) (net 9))
 (segment (start 124.704001 114.040999) (end 135.358799 114.040999) (width 0.25) (layer F.Cu) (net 9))
 (segment (start 123.124 115.621) (end 124.704001 114.040999) (width 0.25) (layer F.Cu) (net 9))
 (segment (start 122.374 115.621) (end 123.124 115.621) (width 0.25) (layer F.Cu) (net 9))
 (segment (start 113.7708 131.762) (end 113.7708 129.761) (width 0.25) (layer F.Cu) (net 1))
 (segment (start 113.7708 132.411) (end 113.7708 132.762) (width 0.25) (layer F.Cu) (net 1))
 (segment (start 115.6708 130.511) (end 113.7708 132.411) (width 0.25) (layer F.Cu) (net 1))
 (segment (start 115.6708 129.761) (end 115.6708 130.511) (width 0.25) (layer F.Cu) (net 1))
 (segment (start 113.7708 136.098) (end 113.7708 132.762) (width 0.25) (layer F.Cu) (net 1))
 (segment (start 113.7708 132.762) (end 113.7708 131.762) (width 0.25) (layer F.Cu) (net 1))
 (segment (start 141.874 124.716) (end 139.64331 124.716) (width 0.25) (layer F.Cu) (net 54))
 (segment (start 118.044 115.621) (end 117.294 115.621) (width 0.25) (layer F.Cu) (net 8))
 (segment (start 119.864 117.441) (end 118.044 115.621) (width 0.25) (layer F.Cu) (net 8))
 (segment (start 119.864 120.756) (end 119.864 117.441) (width 0.25) (layer F.Cu) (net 8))
 (segment (start 131.8588 115.621) (end 132.6088 115.621) (width 0.25) (layer F.Cu) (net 8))
 (segment (start 125.749 115.621) (end 131.8588 115.621) (width 0.25) (layer F.Cu) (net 8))
 (segment (start 120.614 120.756) (end 125.749 115.621) (width 0.25) (layer F.Cu) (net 8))
 (segment (start 119.864 120.756) (end 120.614 120.756) (width 0.25) (layer F.Cu) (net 8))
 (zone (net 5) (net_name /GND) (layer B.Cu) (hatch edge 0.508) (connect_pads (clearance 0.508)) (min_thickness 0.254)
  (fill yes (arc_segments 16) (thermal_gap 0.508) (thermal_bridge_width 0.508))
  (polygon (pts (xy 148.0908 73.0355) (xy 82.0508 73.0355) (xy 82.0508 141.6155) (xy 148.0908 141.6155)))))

